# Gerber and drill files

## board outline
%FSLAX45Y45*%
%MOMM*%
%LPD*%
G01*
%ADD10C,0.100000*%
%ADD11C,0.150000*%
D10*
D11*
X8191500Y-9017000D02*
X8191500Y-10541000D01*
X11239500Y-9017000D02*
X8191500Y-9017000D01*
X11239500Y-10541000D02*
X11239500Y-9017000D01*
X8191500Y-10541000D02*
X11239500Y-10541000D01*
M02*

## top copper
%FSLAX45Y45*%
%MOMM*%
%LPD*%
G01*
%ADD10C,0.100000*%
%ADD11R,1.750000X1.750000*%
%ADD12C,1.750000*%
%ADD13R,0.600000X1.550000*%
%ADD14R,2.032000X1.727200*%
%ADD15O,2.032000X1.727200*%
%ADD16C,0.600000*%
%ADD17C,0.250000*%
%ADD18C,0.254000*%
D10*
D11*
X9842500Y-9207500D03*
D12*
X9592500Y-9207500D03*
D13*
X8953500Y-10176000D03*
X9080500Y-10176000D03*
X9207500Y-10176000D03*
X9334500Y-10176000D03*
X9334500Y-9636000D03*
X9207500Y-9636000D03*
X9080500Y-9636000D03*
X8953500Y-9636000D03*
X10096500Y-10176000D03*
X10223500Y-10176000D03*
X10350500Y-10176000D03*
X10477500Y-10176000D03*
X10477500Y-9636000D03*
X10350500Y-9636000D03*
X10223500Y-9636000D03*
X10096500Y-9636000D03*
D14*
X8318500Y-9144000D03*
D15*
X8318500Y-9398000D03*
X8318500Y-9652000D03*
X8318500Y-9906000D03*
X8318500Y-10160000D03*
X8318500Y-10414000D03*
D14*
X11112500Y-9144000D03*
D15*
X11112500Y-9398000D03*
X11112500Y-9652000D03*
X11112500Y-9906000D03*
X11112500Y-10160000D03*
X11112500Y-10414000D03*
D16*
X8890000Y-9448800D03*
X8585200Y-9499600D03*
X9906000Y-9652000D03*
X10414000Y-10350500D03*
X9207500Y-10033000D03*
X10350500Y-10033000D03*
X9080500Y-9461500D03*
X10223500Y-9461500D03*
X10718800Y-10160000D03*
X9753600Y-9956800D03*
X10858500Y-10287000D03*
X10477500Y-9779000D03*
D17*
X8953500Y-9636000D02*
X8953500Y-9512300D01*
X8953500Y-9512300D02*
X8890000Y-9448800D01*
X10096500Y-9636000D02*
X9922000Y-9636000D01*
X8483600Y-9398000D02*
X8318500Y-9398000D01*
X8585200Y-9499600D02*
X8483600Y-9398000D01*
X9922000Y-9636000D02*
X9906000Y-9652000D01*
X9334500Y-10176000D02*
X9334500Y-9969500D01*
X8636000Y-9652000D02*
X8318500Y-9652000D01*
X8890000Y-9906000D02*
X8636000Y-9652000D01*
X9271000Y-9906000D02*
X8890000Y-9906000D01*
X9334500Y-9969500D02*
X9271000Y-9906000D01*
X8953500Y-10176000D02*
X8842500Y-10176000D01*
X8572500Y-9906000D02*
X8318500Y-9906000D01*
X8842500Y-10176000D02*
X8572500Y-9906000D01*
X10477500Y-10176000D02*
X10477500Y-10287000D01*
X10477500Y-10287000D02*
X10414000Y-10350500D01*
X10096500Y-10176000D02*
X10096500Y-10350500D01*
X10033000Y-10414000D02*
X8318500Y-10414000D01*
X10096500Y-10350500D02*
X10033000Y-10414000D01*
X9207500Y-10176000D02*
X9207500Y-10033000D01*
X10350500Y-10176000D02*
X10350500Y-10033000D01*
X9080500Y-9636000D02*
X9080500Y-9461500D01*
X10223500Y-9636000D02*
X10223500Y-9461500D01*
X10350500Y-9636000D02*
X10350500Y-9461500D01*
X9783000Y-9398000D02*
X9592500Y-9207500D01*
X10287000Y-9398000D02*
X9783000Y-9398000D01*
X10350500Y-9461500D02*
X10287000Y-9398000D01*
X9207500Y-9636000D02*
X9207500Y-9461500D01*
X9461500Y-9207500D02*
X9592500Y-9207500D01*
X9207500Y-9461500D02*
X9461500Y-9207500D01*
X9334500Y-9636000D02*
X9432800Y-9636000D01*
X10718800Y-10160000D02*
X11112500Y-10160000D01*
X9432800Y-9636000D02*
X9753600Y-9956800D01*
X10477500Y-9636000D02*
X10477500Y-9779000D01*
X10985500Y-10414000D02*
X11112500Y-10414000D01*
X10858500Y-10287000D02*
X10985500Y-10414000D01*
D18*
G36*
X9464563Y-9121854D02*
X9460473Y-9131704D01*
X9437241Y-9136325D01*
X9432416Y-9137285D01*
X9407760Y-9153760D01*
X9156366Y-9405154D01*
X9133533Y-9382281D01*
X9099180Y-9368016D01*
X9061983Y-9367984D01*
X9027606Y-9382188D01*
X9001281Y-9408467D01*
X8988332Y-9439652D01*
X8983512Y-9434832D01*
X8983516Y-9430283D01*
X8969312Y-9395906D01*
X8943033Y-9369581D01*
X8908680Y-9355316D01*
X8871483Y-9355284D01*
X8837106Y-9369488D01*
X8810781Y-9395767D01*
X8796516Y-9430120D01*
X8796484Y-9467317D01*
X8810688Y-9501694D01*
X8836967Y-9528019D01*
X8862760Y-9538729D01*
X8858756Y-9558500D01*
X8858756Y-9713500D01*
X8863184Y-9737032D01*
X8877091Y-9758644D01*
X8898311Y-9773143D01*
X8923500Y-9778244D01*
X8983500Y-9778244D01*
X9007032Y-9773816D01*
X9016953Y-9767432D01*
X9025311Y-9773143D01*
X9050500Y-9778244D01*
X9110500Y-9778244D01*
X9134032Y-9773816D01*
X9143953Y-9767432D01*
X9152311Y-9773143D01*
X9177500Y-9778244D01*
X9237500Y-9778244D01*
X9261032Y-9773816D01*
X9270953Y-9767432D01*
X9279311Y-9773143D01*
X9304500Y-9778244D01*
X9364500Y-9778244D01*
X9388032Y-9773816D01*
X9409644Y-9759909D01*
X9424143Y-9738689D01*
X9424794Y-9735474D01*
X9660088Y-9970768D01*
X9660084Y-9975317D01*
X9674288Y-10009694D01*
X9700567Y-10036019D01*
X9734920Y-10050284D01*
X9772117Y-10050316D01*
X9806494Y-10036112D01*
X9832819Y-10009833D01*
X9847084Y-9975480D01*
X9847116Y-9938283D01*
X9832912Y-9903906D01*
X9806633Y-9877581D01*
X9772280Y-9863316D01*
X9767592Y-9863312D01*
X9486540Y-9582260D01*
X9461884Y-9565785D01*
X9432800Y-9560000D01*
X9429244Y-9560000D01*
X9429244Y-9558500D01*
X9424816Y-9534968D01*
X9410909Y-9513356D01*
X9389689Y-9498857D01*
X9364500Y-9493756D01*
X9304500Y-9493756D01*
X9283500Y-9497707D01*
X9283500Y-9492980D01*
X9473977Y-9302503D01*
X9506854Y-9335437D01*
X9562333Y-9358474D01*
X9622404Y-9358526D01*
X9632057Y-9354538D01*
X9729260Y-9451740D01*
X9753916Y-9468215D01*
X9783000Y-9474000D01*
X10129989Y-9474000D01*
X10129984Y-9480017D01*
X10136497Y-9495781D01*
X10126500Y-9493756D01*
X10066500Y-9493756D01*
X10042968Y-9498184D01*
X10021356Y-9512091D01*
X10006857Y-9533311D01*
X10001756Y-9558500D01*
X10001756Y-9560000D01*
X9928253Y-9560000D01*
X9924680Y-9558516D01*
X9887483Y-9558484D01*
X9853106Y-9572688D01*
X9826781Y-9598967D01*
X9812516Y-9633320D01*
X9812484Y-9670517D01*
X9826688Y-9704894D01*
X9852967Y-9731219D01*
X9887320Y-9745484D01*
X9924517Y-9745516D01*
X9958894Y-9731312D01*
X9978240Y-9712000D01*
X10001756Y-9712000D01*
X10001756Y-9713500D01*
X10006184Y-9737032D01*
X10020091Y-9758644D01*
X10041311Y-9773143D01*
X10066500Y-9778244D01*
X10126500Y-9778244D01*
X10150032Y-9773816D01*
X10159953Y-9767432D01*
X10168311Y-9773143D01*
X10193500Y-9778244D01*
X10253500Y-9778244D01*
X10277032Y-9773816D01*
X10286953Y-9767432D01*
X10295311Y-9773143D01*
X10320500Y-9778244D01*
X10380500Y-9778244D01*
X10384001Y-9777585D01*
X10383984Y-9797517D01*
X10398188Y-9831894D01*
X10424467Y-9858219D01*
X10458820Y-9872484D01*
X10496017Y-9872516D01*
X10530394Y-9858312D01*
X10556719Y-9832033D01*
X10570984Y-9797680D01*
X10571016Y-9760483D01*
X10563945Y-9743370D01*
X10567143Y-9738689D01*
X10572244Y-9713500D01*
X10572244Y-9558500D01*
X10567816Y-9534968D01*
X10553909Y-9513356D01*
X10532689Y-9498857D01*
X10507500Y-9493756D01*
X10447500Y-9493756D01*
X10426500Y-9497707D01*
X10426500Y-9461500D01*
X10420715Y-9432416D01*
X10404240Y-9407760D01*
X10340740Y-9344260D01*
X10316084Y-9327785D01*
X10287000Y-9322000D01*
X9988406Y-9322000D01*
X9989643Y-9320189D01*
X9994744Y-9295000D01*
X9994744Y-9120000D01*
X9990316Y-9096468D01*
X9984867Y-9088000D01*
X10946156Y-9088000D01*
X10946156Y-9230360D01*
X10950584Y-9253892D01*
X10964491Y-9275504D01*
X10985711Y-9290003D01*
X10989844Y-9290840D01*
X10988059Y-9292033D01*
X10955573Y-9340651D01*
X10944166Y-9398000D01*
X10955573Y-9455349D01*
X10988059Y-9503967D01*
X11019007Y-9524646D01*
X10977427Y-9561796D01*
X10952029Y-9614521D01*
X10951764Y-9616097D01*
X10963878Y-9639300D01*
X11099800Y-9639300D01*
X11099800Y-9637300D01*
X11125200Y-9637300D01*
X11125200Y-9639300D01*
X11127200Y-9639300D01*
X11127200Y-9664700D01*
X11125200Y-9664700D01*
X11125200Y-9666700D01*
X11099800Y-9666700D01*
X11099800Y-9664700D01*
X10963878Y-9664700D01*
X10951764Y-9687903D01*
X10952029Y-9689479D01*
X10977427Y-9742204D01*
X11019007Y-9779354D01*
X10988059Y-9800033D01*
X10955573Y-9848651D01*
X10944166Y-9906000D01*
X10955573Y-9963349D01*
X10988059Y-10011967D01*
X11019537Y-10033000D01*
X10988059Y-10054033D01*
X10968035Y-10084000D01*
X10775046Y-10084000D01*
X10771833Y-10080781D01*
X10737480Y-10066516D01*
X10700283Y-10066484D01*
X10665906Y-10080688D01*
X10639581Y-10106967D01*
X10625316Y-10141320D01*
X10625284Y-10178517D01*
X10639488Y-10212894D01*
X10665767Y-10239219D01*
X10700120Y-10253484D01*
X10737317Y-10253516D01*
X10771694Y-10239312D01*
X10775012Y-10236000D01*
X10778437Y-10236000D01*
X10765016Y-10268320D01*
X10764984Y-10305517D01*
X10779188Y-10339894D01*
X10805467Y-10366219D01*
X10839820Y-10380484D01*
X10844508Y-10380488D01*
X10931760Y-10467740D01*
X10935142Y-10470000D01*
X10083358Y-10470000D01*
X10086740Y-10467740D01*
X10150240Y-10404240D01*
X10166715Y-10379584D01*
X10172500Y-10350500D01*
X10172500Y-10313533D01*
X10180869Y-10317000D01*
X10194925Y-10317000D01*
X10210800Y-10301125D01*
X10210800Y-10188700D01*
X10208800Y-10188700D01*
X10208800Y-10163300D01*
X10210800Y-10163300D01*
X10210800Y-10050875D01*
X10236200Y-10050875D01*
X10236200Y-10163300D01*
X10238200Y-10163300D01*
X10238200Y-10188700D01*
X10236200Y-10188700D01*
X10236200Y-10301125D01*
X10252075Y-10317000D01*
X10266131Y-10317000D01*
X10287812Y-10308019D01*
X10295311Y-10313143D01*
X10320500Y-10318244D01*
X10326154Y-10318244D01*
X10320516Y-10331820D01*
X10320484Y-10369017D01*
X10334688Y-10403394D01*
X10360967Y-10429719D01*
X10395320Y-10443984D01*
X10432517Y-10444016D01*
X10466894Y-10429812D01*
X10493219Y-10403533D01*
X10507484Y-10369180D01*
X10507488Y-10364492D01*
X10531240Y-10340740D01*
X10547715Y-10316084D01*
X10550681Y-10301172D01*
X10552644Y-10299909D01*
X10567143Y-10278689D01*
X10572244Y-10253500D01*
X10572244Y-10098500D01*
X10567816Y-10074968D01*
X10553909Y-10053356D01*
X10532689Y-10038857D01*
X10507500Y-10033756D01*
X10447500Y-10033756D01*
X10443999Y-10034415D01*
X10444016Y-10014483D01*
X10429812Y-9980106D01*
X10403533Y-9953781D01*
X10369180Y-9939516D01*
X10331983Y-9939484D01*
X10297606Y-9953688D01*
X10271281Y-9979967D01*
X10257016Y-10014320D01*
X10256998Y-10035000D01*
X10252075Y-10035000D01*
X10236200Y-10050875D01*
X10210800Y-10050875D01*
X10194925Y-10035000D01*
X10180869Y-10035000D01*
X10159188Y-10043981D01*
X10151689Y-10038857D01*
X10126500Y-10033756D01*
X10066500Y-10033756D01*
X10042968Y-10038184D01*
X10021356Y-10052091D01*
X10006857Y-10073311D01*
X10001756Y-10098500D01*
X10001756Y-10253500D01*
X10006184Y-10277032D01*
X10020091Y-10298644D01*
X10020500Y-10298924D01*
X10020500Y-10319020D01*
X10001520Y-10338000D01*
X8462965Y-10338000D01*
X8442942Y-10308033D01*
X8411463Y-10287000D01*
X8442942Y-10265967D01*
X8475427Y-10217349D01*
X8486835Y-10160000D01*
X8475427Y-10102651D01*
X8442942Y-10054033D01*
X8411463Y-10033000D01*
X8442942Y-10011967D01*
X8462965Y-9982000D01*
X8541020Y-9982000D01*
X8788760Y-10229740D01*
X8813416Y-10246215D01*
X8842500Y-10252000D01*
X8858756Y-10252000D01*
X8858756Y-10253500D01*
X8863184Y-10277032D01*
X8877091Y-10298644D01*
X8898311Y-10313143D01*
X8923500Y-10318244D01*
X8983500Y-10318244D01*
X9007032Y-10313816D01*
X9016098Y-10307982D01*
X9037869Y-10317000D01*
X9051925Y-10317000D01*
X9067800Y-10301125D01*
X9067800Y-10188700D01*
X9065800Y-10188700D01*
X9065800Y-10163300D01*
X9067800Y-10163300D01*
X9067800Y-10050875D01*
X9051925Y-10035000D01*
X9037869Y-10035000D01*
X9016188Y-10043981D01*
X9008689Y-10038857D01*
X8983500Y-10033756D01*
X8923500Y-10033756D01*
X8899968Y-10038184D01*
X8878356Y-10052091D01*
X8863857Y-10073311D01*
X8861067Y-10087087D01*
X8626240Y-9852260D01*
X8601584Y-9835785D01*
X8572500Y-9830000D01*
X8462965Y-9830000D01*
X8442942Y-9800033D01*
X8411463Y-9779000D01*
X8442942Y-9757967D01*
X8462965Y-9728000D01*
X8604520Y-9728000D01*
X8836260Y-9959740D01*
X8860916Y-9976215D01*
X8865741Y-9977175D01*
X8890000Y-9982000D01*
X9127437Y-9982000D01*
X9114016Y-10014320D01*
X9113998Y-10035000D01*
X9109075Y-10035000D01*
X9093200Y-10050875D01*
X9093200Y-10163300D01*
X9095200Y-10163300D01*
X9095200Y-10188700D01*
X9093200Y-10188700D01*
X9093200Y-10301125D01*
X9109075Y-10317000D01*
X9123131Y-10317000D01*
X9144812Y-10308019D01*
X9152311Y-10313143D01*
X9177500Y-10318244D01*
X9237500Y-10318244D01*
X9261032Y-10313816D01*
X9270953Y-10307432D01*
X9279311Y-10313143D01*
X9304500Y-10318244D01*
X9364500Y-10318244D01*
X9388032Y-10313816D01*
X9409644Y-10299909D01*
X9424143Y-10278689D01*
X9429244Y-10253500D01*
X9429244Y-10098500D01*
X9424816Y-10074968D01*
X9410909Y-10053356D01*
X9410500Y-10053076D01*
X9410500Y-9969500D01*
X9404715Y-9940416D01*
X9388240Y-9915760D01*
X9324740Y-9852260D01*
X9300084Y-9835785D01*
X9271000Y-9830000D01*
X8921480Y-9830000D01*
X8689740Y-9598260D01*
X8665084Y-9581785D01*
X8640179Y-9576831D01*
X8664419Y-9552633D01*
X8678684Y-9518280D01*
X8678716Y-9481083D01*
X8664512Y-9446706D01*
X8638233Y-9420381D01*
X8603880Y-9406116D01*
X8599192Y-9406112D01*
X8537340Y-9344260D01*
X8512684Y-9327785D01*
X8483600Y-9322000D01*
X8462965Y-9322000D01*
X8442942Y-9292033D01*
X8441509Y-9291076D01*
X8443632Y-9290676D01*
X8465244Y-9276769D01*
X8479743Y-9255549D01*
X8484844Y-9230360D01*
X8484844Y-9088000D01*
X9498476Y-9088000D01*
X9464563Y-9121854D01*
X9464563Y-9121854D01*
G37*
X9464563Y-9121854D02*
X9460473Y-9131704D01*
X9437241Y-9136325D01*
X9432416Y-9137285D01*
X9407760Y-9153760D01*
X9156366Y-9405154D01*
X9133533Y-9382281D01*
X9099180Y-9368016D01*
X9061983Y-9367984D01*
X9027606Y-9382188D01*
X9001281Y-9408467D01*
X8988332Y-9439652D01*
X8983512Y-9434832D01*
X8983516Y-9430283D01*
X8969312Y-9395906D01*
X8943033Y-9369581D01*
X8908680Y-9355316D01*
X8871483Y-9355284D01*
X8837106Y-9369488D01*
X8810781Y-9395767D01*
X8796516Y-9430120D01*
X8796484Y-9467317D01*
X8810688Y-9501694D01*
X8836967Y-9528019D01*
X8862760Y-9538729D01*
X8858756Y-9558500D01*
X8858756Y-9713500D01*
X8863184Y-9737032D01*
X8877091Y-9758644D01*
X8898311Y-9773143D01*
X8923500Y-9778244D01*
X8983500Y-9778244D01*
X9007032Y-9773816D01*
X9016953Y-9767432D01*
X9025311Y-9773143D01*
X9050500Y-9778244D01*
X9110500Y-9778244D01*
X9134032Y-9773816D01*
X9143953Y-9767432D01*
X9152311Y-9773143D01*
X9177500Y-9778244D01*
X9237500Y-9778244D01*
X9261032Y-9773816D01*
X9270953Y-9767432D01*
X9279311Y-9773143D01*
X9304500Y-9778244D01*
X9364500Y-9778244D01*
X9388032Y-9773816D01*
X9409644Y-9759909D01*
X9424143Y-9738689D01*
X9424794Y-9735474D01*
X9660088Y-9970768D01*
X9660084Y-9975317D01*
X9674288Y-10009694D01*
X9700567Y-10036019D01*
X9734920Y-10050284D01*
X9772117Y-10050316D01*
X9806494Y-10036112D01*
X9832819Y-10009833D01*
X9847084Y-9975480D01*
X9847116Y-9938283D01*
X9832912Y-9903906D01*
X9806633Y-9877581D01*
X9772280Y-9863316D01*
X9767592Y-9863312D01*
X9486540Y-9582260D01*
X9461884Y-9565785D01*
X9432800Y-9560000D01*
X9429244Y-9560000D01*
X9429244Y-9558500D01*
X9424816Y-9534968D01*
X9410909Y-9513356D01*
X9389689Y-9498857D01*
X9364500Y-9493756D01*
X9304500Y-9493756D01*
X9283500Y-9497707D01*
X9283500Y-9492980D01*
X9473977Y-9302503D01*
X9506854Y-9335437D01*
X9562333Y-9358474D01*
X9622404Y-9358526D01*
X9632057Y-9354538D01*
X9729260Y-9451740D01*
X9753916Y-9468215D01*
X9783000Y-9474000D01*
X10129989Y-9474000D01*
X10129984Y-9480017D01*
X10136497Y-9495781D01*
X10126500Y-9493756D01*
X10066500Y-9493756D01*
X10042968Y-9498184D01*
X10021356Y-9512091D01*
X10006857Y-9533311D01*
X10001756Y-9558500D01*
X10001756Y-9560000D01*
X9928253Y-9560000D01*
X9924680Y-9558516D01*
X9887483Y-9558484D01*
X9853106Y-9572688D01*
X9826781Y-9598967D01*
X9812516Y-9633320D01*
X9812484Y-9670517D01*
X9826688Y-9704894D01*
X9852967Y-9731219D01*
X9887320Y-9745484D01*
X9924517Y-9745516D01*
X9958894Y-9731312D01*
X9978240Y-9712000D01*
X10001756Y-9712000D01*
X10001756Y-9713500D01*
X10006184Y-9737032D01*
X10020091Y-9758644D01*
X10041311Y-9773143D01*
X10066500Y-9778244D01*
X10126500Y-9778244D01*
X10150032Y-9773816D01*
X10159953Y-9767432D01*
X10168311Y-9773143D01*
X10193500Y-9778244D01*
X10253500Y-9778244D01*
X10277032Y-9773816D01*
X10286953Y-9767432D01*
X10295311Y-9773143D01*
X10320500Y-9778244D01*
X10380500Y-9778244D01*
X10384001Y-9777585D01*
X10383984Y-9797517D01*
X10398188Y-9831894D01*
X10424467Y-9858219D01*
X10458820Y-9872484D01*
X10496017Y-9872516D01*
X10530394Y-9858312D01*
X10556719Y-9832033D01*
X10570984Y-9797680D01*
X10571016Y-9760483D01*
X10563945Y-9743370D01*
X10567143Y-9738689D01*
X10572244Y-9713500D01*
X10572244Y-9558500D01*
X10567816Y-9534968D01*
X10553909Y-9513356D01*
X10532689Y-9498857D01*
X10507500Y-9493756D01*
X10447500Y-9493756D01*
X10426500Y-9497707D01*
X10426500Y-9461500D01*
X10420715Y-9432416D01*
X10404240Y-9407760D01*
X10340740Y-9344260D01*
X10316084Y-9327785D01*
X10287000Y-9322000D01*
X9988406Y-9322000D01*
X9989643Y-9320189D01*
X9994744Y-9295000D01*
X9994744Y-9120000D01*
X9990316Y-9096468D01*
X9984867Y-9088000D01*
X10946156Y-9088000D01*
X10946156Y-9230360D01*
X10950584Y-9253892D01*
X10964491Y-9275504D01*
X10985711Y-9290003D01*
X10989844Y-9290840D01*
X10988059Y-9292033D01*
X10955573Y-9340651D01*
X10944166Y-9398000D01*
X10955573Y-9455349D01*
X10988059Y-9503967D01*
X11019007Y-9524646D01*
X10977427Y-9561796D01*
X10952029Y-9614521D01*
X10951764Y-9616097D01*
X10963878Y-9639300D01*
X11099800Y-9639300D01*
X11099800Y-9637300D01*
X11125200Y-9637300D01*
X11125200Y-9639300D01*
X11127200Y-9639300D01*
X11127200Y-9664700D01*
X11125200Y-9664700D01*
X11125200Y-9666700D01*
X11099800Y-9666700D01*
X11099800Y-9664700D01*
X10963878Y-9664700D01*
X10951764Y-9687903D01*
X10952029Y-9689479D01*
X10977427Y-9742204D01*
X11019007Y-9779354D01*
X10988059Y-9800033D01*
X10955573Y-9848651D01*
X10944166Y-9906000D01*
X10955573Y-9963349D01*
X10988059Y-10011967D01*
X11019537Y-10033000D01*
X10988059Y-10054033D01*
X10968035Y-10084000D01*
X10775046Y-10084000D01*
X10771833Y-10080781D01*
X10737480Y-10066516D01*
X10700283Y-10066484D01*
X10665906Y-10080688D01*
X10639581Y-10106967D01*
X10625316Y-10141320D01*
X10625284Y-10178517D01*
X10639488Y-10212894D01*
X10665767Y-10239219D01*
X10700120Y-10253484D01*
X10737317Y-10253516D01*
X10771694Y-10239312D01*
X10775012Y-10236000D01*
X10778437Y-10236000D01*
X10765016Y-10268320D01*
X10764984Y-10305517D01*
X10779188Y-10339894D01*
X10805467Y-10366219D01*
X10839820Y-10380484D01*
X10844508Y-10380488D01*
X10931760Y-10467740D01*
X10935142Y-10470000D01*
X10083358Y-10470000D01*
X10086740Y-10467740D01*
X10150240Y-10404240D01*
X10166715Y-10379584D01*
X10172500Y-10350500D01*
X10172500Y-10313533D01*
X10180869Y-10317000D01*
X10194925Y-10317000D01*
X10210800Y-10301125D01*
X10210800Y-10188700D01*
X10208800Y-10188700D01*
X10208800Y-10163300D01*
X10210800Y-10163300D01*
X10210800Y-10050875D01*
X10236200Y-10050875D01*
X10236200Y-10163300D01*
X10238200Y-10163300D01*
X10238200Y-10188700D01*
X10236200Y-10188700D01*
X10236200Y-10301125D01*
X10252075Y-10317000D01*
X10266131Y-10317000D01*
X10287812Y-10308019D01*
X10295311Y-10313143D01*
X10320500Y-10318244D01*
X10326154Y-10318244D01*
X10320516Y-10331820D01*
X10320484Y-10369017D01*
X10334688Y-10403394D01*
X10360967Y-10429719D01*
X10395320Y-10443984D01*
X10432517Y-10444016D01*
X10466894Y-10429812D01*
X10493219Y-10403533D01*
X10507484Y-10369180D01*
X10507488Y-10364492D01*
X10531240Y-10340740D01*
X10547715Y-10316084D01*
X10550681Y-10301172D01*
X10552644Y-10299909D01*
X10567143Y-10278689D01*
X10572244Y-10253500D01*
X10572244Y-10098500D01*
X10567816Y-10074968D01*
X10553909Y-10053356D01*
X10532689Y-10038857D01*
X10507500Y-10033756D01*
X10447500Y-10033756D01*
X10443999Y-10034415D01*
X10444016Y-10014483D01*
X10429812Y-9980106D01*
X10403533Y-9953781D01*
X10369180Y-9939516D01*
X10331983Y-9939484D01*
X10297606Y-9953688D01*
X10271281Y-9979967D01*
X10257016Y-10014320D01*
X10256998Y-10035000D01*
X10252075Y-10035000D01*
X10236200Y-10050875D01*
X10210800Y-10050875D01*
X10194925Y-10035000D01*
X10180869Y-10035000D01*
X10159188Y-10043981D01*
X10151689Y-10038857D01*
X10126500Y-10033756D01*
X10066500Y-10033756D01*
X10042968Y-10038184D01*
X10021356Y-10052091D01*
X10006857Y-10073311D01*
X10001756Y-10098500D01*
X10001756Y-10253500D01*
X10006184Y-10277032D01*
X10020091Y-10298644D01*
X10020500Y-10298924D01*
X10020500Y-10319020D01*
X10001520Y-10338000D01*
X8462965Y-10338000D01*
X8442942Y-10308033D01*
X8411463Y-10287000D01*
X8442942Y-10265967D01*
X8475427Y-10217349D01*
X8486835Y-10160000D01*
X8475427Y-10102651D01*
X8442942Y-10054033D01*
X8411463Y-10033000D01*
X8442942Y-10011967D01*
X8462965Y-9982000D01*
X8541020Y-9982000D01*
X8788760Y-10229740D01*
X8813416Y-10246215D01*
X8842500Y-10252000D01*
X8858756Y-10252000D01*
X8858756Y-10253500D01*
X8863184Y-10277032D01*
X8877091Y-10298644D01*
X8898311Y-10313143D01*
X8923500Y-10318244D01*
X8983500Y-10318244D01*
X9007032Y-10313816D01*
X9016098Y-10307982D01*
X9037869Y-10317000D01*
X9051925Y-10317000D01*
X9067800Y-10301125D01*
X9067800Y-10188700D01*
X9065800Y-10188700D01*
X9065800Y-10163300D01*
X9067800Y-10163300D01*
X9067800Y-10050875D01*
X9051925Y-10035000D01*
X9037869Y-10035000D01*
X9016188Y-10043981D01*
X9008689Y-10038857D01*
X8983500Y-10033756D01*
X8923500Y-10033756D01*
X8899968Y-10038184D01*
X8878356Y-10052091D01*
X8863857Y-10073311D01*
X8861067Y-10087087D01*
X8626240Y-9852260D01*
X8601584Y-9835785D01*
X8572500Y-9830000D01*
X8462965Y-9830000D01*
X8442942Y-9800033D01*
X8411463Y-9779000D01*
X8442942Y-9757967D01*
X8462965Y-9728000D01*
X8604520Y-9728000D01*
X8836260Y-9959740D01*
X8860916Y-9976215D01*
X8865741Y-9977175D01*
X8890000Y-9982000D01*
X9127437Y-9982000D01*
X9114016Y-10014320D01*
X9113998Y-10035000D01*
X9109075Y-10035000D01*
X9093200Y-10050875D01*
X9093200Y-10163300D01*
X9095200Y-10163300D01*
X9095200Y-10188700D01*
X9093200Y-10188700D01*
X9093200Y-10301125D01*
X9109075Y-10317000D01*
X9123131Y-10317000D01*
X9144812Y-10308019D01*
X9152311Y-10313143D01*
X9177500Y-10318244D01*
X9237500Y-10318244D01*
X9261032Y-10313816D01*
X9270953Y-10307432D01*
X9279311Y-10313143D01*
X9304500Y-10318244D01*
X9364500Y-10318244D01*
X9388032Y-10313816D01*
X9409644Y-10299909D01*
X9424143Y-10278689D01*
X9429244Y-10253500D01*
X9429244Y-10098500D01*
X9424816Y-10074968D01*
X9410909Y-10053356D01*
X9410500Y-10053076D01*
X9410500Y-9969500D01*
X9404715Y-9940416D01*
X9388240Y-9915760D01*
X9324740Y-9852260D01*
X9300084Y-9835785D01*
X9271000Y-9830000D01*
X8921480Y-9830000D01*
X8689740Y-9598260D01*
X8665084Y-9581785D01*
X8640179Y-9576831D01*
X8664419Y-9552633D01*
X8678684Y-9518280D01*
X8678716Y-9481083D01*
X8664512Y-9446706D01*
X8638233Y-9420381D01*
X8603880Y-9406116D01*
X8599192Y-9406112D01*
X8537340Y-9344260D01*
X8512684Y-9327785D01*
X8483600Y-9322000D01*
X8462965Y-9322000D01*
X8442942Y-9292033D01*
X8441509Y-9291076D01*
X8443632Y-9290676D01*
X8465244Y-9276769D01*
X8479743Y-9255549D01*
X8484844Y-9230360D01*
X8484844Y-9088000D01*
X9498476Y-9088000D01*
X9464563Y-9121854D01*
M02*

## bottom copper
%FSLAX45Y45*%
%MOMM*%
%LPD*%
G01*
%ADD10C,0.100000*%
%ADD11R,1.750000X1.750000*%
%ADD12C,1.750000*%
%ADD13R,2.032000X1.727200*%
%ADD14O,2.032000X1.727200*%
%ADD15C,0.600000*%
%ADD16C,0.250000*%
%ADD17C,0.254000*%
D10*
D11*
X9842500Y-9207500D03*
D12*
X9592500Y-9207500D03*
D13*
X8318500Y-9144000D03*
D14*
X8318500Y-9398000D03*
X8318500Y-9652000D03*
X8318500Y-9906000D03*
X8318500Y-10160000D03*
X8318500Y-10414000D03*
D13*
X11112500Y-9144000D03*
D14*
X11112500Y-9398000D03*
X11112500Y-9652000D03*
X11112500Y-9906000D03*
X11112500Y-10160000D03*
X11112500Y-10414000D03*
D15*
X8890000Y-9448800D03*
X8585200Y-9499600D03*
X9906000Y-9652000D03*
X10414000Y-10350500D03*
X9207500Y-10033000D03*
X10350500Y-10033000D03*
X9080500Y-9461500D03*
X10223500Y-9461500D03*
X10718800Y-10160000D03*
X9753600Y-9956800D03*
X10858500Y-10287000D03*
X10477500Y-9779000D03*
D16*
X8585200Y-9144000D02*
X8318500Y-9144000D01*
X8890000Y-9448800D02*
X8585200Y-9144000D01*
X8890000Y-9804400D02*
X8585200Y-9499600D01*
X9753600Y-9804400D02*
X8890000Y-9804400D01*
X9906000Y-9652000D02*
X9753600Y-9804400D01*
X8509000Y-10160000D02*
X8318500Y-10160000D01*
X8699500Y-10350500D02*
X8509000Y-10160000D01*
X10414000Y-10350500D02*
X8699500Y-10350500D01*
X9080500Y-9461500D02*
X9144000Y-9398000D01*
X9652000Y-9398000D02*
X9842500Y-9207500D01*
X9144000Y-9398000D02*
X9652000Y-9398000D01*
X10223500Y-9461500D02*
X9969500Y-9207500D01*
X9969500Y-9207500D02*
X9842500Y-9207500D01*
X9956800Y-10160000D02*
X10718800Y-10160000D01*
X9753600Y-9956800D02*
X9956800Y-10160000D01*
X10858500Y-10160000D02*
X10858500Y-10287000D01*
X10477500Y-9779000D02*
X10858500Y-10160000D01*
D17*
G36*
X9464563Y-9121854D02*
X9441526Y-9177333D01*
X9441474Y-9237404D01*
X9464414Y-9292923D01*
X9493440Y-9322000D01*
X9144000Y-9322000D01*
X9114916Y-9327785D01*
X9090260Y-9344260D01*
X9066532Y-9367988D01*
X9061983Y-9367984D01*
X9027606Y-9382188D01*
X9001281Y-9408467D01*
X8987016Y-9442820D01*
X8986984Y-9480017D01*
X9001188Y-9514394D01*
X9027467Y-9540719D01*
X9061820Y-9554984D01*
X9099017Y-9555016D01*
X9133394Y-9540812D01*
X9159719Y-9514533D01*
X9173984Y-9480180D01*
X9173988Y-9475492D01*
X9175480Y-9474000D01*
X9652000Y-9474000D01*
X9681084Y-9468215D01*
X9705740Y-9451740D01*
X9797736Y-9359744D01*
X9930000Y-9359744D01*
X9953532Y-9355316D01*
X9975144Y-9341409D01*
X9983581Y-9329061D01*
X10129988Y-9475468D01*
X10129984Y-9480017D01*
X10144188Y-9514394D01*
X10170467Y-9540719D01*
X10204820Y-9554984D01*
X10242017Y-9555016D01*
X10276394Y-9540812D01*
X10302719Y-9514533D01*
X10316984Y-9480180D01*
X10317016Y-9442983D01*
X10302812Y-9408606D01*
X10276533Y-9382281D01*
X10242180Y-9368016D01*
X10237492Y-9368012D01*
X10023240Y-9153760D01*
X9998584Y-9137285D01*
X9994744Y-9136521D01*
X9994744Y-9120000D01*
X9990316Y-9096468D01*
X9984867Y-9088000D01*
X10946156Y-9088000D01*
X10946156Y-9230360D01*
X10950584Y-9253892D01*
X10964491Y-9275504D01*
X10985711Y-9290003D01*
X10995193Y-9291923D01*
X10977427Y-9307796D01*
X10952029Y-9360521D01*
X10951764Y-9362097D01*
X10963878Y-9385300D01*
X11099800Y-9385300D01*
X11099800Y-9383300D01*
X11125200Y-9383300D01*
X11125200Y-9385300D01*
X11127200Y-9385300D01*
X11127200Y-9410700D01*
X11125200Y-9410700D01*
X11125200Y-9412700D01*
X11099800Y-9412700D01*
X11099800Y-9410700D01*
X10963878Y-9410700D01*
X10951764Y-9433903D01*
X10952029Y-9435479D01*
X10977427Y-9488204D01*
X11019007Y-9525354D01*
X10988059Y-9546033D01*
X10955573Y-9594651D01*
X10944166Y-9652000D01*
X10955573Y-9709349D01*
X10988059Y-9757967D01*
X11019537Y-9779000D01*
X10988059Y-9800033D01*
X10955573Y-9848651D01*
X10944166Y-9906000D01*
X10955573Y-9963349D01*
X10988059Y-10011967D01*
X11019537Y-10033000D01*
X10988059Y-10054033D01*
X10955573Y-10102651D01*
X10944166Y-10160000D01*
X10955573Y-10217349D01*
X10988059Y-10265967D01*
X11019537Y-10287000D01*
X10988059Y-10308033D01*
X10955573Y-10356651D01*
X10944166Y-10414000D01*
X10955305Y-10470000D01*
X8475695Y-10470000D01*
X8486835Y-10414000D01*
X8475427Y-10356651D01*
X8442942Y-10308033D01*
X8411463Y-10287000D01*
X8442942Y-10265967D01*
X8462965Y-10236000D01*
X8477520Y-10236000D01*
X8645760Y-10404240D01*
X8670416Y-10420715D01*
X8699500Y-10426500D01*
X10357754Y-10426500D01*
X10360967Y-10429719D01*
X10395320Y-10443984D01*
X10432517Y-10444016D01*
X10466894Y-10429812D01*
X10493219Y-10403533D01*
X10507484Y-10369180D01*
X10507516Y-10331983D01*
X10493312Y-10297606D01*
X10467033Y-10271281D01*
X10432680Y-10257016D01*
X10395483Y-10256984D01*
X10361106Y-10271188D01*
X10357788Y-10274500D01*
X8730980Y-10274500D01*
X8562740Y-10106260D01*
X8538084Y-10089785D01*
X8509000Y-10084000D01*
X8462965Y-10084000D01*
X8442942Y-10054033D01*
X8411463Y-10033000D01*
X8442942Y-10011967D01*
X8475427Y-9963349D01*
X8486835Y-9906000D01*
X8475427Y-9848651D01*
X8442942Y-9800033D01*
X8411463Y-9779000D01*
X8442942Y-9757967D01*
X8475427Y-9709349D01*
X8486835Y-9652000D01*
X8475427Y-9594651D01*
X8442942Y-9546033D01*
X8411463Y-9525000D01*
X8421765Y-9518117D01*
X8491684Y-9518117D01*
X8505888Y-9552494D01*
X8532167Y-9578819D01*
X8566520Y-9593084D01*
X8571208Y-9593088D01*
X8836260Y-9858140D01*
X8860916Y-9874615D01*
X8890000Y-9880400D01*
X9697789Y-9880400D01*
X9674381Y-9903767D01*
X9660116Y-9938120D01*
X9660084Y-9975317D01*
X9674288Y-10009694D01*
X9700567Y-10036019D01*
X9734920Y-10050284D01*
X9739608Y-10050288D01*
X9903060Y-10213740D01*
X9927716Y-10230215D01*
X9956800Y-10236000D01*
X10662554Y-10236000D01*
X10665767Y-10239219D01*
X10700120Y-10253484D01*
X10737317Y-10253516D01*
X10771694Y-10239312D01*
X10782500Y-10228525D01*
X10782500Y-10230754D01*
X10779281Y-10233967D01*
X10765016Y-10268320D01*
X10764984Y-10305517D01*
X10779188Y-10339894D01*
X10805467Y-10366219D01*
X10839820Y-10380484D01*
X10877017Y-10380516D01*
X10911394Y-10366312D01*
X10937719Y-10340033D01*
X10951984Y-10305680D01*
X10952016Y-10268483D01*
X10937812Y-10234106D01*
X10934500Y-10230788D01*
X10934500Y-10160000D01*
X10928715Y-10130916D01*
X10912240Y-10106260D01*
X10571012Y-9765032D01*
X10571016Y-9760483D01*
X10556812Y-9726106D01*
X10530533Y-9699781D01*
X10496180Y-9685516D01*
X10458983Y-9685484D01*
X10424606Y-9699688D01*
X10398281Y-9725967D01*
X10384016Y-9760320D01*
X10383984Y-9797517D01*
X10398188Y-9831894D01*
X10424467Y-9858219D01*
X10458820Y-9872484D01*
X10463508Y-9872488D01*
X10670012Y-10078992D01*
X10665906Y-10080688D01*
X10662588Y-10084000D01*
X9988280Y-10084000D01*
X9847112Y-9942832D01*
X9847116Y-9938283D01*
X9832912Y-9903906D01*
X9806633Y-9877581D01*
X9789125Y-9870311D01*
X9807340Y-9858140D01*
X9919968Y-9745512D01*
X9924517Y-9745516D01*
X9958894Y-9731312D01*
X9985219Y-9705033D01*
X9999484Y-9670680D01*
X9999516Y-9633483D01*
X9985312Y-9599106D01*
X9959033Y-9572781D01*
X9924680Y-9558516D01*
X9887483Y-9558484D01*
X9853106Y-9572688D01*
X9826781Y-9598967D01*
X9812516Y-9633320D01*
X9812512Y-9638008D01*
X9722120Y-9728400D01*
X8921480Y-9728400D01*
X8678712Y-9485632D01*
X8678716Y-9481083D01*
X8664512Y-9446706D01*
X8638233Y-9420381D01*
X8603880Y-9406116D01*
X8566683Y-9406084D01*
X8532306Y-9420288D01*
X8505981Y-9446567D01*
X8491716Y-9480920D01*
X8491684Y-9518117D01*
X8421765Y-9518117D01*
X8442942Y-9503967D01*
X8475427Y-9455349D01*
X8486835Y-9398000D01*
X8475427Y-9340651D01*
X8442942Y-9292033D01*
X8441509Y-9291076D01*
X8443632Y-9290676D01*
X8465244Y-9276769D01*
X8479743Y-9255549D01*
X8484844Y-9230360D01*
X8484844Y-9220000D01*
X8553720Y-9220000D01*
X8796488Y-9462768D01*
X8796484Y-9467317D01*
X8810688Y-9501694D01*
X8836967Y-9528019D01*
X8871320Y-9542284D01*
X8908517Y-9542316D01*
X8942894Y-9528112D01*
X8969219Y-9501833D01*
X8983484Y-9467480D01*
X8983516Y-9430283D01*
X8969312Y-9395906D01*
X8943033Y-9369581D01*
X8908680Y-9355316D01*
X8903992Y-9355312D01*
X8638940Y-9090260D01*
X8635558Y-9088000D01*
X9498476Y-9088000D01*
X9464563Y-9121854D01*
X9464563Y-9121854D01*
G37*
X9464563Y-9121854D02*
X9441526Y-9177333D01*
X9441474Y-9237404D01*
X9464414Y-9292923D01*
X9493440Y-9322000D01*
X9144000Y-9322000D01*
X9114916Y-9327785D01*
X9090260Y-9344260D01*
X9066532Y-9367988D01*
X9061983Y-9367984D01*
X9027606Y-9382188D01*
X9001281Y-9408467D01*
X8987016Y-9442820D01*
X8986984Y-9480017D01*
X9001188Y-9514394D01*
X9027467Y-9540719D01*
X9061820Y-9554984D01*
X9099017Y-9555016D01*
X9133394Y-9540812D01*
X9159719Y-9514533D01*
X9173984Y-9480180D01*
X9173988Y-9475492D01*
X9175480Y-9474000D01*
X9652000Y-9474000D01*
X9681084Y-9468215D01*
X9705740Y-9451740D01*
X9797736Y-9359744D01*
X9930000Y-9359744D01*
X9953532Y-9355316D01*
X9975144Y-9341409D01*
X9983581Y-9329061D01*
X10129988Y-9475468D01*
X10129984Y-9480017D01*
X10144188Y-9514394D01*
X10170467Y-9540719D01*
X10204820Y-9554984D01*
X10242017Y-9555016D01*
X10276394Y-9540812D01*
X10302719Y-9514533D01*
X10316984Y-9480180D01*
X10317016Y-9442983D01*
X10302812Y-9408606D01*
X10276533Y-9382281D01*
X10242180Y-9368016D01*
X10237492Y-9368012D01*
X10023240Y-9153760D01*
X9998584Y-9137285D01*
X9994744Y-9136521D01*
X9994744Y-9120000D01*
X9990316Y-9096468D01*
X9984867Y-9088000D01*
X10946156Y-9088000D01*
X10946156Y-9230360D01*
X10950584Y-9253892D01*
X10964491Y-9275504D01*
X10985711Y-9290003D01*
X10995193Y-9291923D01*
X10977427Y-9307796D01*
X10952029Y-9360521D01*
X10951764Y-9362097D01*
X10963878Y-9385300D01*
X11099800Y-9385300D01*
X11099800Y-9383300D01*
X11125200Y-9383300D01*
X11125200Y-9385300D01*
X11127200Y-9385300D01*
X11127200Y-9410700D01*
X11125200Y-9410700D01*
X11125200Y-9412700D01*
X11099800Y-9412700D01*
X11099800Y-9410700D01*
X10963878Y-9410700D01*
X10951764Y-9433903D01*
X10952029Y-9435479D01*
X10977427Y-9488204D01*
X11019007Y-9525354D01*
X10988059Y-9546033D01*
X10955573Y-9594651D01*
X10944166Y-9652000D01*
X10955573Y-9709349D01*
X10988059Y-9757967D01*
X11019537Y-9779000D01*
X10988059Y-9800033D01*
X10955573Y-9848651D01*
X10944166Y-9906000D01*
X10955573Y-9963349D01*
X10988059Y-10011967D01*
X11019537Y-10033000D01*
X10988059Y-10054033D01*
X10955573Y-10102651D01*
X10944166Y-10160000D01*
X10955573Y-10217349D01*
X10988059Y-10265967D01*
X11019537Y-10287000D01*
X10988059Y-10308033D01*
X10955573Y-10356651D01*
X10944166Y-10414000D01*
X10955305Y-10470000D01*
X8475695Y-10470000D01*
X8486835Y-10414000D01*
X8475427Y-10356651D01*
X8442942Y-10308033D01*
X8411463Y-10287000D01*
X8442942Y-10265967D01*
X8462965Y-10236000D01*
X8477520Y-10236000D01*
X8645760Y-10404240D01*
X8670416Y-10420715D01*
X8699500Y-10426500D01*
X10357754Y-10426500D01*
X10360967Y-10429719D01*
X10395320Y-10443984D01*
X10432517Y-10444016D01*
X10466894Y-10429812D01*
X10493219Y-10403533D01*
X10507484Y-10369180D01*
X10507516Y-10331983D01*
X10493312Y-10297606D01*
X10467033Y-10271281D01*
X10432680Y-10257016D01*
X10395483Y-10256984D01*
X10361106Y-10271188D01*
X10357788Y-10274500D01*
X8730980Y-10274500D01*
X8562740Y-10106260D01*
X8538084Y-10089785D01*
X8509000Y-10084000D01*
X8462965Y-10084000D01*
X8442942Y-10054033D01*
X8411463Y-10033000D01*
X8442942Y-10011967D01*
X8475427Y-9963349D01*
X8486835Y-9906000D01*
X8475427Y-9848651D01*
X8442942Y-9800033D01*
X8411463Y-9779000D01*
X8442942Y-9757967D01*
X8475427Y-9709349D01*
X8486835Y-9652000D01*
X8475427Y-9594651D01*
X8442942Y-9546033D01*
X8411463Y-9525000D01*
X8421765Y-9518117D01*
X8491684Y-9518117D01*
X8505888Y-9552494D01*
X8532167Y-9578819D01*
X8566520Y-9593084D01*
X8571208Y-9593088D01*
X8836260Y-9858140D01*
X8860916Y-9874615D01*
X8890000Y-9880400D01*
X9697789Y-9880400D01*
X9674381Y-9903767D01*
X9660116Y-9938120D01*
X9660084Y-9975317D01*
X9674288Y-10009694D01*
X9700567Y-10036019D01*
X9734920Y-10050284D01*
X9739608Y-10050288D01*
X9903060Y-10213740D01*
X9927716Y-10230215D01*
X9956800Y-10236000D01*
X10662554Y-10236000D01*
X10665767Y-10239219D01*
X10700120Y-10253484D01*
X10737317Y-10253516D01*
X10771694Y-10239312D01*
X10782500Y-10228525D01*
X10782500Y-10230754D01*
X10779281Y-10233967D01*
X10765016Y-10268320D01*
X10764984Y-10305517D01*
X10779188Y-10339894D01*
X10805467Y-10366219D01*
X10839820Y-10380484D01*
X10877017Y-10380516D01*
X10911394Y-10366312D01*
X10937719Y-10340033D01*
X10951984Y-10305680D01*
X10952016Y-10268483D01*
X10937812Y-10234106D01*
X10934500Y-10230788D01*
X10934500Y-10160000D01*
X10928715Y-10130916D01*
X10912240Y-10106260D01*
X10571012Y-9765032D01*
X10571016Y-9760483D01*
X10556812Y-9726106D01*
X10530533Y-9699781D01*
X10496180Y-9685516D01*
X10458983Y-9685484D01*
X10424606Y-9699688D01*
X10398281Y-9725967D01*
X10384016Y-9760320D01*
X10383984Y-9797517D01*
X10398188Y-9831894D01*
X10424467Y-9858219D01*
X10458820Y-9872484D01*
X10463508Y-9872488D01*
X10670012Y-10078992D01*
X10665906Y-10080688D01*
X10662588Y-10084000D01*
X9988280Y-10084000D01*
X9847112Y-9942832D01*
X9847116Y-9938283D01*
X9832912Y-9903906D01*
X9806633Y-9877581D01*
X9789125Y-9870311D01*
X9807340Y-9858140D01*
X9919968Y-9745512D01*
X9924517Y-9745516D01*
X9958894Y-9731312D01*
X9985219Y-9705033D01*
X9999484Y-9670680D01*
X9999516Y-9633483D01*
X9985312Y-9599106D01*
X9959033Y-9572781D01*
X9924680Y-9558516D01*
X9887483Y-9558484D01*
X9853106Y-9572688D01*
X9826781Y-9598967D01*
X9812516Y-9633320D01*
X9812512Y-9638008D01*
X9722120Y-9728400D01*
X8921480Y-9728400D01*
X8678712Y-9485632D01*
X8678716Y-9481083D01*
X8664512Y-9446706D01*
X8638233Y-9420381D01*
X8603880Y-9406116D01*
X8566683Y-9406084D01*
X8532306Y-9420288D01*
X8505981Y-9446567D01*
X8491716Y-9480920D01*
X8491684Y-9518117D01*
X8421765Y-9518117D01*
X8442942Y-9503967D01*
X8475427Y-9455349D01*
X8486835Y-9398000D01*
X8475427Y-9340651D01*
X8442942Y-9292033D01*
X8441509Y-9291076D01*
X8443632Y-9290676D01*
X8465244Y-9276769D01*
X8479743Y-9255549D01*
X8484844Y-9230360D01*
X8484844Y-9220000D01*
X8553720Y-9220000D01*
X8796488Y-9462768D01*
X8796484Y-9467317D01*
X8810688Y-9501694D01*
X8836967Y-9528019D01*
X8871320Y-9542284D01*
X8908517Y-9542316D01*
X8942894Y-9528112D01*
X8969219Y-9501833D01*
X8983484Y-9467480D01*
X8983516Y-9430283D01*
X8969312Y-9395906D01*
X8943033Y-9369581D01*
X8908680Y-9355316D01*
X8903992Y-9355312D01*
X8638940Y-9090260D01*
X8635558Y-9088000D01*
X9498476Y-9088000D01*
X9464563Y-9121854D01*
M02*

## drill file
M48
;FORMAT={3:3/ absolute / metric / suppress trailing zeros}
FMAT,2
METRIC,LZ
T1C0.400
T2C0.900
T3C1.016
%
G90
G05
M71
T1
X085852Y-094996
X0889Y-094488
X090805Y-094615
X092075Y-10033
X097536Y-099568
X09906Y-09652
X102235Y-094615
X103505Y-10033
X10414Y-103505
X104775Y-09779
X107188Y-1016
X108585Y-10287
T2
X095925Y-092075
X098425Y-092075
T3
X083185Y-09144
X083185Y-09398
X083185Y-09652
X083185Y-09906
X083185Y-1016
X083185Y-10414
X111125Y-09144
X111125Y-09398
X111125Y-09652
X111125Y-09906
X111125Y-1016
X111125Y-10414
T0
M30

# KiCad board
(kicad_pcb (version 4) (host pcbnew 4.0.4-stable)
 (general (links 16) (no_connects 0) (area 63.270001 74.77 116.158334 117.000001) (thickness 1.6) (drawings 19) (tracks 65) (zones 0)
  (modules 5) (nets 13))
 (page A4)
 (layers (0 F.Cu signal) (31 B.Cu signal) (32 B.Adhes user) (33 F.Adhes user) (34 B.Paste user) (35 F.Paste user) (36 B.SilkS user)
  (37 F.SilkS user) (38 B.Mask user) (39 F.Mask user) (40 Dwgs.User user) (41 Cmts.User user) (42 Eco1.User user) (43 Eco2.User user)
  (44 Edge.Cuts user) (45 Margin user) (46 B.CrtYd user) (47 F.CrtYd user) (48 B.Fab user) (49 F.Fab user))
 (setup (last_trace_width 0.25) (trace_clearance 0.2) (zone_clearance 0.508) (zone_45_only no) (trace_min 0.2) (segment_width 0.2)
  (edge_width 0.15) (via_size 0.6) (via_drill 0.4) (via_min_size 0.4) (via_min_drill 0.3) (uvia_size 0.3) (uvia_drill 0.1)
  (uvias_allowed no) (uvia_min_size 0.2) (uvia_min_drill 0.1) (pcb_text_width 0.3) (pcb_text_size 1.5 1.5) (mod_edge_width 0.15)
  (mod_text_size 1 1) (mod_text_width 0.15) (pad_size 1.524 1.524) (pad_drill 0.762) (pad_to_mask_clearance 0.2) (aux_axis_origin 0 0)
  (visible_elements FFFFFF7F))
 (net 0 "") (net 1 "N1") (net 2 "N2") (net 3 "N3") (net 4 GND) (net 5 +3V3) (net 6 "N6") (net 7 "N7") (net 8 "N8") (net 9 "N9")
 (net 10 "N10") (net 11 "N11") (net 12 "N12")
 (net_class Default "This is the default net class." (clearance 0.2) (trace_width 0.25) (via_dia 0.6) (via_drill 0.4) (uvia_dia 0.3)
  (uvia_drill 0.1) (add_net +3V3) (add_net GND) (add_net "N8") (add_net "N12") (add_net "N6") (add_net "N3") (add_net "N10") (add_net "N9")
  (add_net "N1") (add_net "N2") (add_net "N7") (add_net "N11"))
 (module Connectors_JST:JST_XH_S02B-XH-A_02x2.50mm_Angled (layer F.Cu) (at 98.425 92.075 180)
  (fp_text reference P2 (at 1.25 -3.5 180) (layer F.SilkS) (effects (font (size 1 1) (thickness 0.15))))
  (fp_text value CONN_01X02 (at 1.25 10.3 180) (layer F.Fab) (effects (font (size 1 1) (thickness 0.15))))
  (pad 1 thru_hole rect (at 0 0 180) (size 1.75 1.75) (drill 0.9) (layers *.Cu *.Mask F.SilkS) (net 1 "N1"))
  (pad 2 thru_hole circle (at 2.5 0 180) (size 1.75 1.75) (drill 0.9) (layers *.Cu *.Mask F.SilkS) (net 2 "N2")))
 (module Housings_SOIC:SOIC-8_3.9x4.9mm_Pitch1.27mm (layer F.Cu) (at 91.44 99.06 90)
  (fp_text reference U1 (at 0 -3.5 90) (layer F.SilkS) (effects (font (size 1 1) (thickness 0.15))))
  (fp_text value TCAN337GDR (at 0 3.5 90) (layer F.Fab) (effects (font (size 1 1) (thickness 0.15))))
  (pad 1 smd rect (at -2.7 -1.905 90) (size 1.55 0.6) (layers F.Cu F.Paste F.Mask) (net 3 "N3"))
  (pad 2 smd rect (at -2.7 -0.635 90) (size 1.55 0.6) (layers F.Cu F.Paste F.Mask) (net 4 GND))
  (pad 3 smd rect (at -2.7 0.635 90) (size 1.55 0.6) (layers F.Cu F.Paste F.Mask) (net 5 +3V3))
  (pad 4 smd rect (at -2.7 1.905 90) (size 1.55 0.6) (layers F.Cu F.Paste F.Mask) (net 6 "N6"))
  (pad 5 smd rect (at 2.7 1.905 90) (size 1.55 0.6) (layers F.Cu F.Paste F.Mask) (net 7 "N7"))
  (pad 6 smd rect (at 2.7 0.635 90) (size 1.55 0.6) (layers F.Cu F.Paste F.Mask) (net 2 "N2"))
  (pad 7 smd rect (at 2.7 -0.635 90) (size 1.55 0.6) (layers F.Cu F.Paste F.Mask) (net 1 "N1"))
  (pad 8 smd rect (at 2.7 -1.905 90) (size 1.55 0.6) (layers F.Cu F.Paste F.Mask) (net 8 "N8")))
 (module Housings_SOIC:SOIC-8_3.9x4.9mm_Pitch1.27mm (layer F.Cu) (at 102.87 99.06 90)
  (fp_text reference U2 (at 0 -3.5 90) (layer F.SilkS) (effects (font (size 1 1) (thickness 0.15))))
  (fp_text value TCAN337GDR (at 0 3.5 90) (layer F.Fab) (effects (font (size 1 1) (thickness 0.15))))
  (pad 1 smd rect (at -2.7 -1.905 90) (size 1.55 0.6) (layers F.Cu F.Paste F.Mask) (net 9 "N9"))
  (pad 2 smd rect (at -2.7 -0.635 90) (size 1.55 0.6) (layers F.Cu F.Paste F.Mask) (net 4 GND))
  (pad 3 smd rect (at -2.7 0.635 90) (size 1.55 0.6) (layers F.Cu F.Paste F.Mask) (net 5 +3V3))
  (pad 4 smd rect (at -2.7 1.905 90) (size 1.55 0.6) (layers F.Cu F.Paste F.Mask) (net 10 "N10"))
  (pad 5 smd rect (at 2.7 1.905 90) (size 1.55 0.6) (layers F.Cu F.Paste F.Mask) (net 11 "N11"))
  (pad 6 smd rect (at 2.7 0.635 90) (size 1.55 0.6) (layers F.Cu F.Paste F.Mask) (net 2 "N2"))
  (pad 7 smd rect (at 2.7 -0.635 90) (size 1.55 0.6) (layers F.Cu F.Paste F.Mask) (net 1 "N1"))
  (pad 8 smd rect (at 2.7 -1.905 90) (size 1.55 0.6) (layers F.Cu F.Paste F.Mask) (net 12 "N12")))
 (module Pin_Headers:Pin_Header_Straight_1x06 (layer F.Cu) (at 83.185 91.44)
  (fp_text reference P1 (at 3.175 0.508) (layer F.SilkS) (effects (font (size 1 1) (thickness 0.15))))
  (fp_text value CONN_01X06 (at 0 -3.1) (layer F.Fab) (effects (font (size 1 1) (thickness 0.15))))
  (pad 1 thru_hole rect (at 0 0) (size 2.032 1.7272) (drill 1.016) (layers *.Cu *.Mask F.SilkS) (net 8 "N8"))
  (pad 2 thru_hole oval (at 0 2.54) (size 2.032 1.7272) (drill 1.016) (layers *.Cu *.Mask F.SilkS) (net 12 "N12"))
  (pad 3 thru_hole oval (at 0 5.08) (size 2.032 1.7272) (drill 1.016) (layers *.Cu *.Mask F.SilkS) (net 6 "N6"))
  (pad 4 thru_hole oval (at 0 7.62) (size 2.032 1.7272) (drill 1.016) (layers *.Cu *.Mask F.SilkS) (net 3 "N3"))
  (pad 5 thru_hole oval (at 0 10.16) (size 2.032 1.7272) (drill 1.016) (layers *.Cu *.Mask F.SilkS) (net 10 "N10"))
  (pad 6 thru_hole oval (at 0 12.7) (size 2.032 1.7272) (drill 1.016) (layers *.Cu *.Mask F.SilkS) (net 9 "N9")))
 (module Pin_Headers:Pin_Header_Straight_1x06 (layer F.Cu) (at 111.125 91.44)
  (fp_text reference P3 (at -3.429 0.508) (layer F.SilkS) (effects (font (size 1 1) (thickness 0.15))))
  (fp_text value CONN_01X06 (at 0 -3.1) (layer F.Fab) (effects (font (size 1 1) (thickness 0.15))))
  (pad 1 thru_hole rect (at 0 0) (size 2.032 1.7272) (drill 1.016) (layers *.Cu *.Mask F.SilkS))
  (pad 2 thru_hole oval (at 0 2.54) (size 2.032 1.7272) (drill 1.016) (layers *.Cu *.Mask F.SilkS) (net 5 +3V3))
  (pad 3 thru_hole oval (at 0 5.08) (size 2.032 1.7272) (drill 1.016) (layers *.Cu *.Mask F.SilkS) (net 4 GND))
  (pad 4 thru_hole oval (at 0 7.62) (size 2.032 1.7272) (drill 1.016) (layers *.Cu *.Mask F.SilkS))
  (pad 5 thru_hole oval (at 0 10.16) (size 2.032 1.7272) (drill 1.016) (layers *.Cu *.Mask F.SilkS) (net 7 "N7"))
  (pad 6 thru_hole oval (at 0 12.7) (size 2.032 1.7272) (drill 1.016) (layers *.Cu *.Mask F.SilkS) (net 11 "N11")))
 (gr_line (start 81.915 90.17) (end 81.915 105.41) (angle 90) (layer Edge.Cuts) (width 0.15))
 (gr_line (start 112.395 90.17) (end 81.915 90.17) (angle 90) (layer Edge.Cuts) (width 0.15))
 (gr_line (start 112.395 105.41) (end 112.395 90.17) (angle 90) (layer Edge.Cuts) (width 0.15))
 (gr_line (start 81.915 105.41) (end 112.395 105.41) (angle 90) (layer Edge.Cuts) (width 0.15))
 (segment (start 89.535 96.36) (end 89.535 95.123) (width 0.25) (layer F.Cu) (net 8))
 (segment (start 85.852 91.44) (end 83.185 91.44) (width 0.25) (layer B.Cu) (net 8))
 (segment (start 88.9 94.488) (end 85.852 91.44) (width 0.25) (layer B.Cu) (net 8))
 (via (at 88.9 94.488) (size 0.6) (drill 0.4) (layers F.Cu B.Cu) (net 8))
 (segment (start 89.535 95.123) (end 88.9 94.488) (width 0.25) (layer F.Cu) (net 8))
 (segment (start 100.965 96.36) (end 99.22 96.36) (width 0.25) (layer F.Cu) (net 12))
 (segment (start 84.836 93.98) (end 83.185 93.98) (width 0.25) (layer F.Cu) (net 12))
 (segment (start 85.852 94.996) (end 84.836 93.98) (width 0.25) (layer F.Cu) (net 12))
 (via (at 85.852 94.996) (size 0.6) (drill 0.4) (layers F.Cu B.Cu) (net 12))
 (segment (start 88.9 98.044) (end 85.852 94.996) (width 0.25) (layer B.Cu) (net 12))
 (segment (start 97.536 98.044) (end 88.9 98.044) (width 0.25) (layer B.Cu) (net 12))
 (segment (start 99.06 96.52) (end 97.536 98.044) (width 0.25) (layer B.Cu) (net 12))
 (via (at 99.06 96.52) (size 0.6) (drill 0.4) (layers F.Cu B.Cu) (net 12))
 (segment (start 99.22 96.36) (end 99.06 96.52) (width 0.25) (layer F.Cu) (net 12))
 (segment (start 93.345 101.76) (end 93.345 99.695) (width 0.25) (layer F.Cu) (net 6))
 (segment (start 86.36 96.52) (end 83.185 96.52) (width 0.25) (layer F.Cu) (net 6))
 (segment (start 88.9 99.06) (end 86.36 96.52) (width 0.25) (layer F.Cu) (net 6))
 (segment (start 92.71 99.06) (end 88.9 99.06) (width 0.25) (layer F.Cu) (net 6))
 (segment (start 93.345 99.695) (end 92.71 99.06) (width 0.25) (layer F.Cu) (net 6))
 (segment (start 89.535 101.76) (end 88.425 101.76) (width 0.25) (layer F.Cu) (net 3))
 (segment (start 85.725 99.06) (end 83.185 99.06) (width 0.25) (layer F.Cu) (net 3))
 (segment (start 88.425 101.76) (end 85.725 99.06) (width 0.25) (layer F.Cu) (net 3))
 (segment (start 104.775 101.76) (end 104.775 102.87) (width 0.25) (layer F.Cu) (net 10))
 (segment (start 85.09 101.6) (end 83.185 101.6) (width 0.25) (layer B.Cu) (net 10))
 (segment (start 86.995 103.505) (end 85.09 101.6) (width 0.25) (layer B.Cu) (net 10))
 (segment (start 104.14 103.505) (end 86.995 103.505) (width 0.25) (layer B.Cu) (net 10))
 (via (at 104.14 103.505) (size 0.6) (drill 0.4) (layers F.Cu B.Cu) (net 10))
 (segment (start 104.775 102.87) (end 104.14 103.505) (width 0.25) (layer F.Cu) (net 10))
 (segment (start 100.965 101.76) (end 100.965 103.505) (width 0.25) (layer F.Cu) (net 9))
 (segment (start 100.33 104.14) (end 83.185 104.14) (width 0.25) (layer F.Cu) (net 9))
 (segment (start 100.965 103.505) (end 100.33 104.14) (width 0.25) (layer F.Cu) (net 9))
 (segment (start 92.075 101.76) (end 92.075 100.33) (width 0.25) (layer F.Cu) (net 5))
 (via (at 92.075 100.33) (size 0.6) (drill 0.4) (layers F.Cu B.Cu) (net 5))
 (segment (start 103.505 101.76) (end 103.505 100.33) (width 0.25) (layer F.Cu) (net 5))
 (via (at 103.505 100.33) (size 0.6) (drill 0.4) (layers F.Cu B.Cu) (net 5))
 (segment (start 90.805 94.615) (end 91.44 93.98) (width 0.25) (layer B.Cu) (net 1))
 (via (at 90.805 94.615) (size 0.6) (drill 0.4) (layers F.Cu B.Cu) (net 1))
 (segment (start 90.805 96.36) (end 90.805 94.615) (width 0.25) (layer F.Cu) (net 1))
 (segment (start 96.52 93.98) (end 98.425 92.075) (width 0.25) (layer B.Cu) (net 1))
 (segment (start 91.44 93.98) (end 96.52 93.98) (width 0.25) (layer B.Cu) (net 1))
 (segment (start 102.235 94.615) (end 99.695 92.075) (width 0.25) (layer B.Cu) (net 1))
 (via (at 102.235 94.615) (size 0.6) (drill 0.4) (layers F.Cu B.Cu) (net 1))
 (segment (start 102.235 96.36) (end 102.235 94.615) (width 0.25) (layer F.Cu) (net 1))
 (segment (start 99.695 92.075) (end 98.425 92.075) (width 0.25) (layer B.Cu) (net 1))
 (segment (start 103.505 96.36) (end 103.505 94.615) (width 0.25) (layer F.Cu) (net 2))
 (segment (start 97.83 93.98) (end 95.925 92.075) (width 0.25) (layer F.Cu) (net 2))
 (segment (start 102.87 93.98) (end 97.83 93.98) (width 0.25) (layer F.Cu) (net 2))
 (segment (start 103.505 94.615) (end 102.87 93.98) (width 0.25) (layer F.Cu) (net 2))
 (segment (start 92.075 96.36) (end 92.075 94.615) (width 0.25) (layer F.Cu) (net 2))
 (segment (start 94.615 92.075) (end 95.925 92.075) (width 0.25) (layer F.Cu) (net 2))
 (segment (start 92.075 94.615) (end 94.615 92.075) (width 0.25) (layer F.Cu) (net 2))
 (segment (start 93.345 96.36) (end 94.328 96.36) (width 0.25) (layer F.Cu) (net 7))
 (segment (start 107.188 101.6) (end 111.125 101.6) (width 0.25) (layer F.Cu) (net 7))
 (via (at 107.188 101.6) (size 0.6) (drill 0.4) (layers F.Cu B.Cu) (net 7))
 (segment (start 99.568 101.6) (end 107.188 101.6) (width 0.25) (layer B.Cu) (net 7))
 (segment (start 97.536 99.568) (end 99.568 101.6) (width 0.25) (layer B.Cu) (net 7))
 (via (at 97.536 99.568) (size 0.6) (drill 0.4) (layers F.Cu B.Cu) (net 7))
 (segment (start 94.328 96.36) (end 97.536 99.568) (width 0.25) (layer F.Cu) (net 7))
 (segment (start 104.775 96.36) (end 104.775 97.79) (width 0.25) (layer F.Cu) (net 11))
 (segment (start 109.855 104.14) (end 111.125 104.14) (width 0.25) (layer F.Cu) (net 11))
 (segment (start 108.585 102.87) (end 109.855 104.14) (width 0.25) (layer F.Cu) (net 11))
 (via (at 108.585 102.87) (size 0.6) (drill 0.4) (layers F.Cu B.Cu) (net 11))
 (segment (start 108.585 101.6) (end 108.585 102.87) (width 0.25) (layer B.Cu) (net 11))
 (segment (start 104.775 97.79) (end 108.585 101.6) (width 0.25) (layer B.Cu) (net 11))
 (via (at 104.775 97.79) (size 0.6) (drill 0.4) (layers F.Cu B.Cu) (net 11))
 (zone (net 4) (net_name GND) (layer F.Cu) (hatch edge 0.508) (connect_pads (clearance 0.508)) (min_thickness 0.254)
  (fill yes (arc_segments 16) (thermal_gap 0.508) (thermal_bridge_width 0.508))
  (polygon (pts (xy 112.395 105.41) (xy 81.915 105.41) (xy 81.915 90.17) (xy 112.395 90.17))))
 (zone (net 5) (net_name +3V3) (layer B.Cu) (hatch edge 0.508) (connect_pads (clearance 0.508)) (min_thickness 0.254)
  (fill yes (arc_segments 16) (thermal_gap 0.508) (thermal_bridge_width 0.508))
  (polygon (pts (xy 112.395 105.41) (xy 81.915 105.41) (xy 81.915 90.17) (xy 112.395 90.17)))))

